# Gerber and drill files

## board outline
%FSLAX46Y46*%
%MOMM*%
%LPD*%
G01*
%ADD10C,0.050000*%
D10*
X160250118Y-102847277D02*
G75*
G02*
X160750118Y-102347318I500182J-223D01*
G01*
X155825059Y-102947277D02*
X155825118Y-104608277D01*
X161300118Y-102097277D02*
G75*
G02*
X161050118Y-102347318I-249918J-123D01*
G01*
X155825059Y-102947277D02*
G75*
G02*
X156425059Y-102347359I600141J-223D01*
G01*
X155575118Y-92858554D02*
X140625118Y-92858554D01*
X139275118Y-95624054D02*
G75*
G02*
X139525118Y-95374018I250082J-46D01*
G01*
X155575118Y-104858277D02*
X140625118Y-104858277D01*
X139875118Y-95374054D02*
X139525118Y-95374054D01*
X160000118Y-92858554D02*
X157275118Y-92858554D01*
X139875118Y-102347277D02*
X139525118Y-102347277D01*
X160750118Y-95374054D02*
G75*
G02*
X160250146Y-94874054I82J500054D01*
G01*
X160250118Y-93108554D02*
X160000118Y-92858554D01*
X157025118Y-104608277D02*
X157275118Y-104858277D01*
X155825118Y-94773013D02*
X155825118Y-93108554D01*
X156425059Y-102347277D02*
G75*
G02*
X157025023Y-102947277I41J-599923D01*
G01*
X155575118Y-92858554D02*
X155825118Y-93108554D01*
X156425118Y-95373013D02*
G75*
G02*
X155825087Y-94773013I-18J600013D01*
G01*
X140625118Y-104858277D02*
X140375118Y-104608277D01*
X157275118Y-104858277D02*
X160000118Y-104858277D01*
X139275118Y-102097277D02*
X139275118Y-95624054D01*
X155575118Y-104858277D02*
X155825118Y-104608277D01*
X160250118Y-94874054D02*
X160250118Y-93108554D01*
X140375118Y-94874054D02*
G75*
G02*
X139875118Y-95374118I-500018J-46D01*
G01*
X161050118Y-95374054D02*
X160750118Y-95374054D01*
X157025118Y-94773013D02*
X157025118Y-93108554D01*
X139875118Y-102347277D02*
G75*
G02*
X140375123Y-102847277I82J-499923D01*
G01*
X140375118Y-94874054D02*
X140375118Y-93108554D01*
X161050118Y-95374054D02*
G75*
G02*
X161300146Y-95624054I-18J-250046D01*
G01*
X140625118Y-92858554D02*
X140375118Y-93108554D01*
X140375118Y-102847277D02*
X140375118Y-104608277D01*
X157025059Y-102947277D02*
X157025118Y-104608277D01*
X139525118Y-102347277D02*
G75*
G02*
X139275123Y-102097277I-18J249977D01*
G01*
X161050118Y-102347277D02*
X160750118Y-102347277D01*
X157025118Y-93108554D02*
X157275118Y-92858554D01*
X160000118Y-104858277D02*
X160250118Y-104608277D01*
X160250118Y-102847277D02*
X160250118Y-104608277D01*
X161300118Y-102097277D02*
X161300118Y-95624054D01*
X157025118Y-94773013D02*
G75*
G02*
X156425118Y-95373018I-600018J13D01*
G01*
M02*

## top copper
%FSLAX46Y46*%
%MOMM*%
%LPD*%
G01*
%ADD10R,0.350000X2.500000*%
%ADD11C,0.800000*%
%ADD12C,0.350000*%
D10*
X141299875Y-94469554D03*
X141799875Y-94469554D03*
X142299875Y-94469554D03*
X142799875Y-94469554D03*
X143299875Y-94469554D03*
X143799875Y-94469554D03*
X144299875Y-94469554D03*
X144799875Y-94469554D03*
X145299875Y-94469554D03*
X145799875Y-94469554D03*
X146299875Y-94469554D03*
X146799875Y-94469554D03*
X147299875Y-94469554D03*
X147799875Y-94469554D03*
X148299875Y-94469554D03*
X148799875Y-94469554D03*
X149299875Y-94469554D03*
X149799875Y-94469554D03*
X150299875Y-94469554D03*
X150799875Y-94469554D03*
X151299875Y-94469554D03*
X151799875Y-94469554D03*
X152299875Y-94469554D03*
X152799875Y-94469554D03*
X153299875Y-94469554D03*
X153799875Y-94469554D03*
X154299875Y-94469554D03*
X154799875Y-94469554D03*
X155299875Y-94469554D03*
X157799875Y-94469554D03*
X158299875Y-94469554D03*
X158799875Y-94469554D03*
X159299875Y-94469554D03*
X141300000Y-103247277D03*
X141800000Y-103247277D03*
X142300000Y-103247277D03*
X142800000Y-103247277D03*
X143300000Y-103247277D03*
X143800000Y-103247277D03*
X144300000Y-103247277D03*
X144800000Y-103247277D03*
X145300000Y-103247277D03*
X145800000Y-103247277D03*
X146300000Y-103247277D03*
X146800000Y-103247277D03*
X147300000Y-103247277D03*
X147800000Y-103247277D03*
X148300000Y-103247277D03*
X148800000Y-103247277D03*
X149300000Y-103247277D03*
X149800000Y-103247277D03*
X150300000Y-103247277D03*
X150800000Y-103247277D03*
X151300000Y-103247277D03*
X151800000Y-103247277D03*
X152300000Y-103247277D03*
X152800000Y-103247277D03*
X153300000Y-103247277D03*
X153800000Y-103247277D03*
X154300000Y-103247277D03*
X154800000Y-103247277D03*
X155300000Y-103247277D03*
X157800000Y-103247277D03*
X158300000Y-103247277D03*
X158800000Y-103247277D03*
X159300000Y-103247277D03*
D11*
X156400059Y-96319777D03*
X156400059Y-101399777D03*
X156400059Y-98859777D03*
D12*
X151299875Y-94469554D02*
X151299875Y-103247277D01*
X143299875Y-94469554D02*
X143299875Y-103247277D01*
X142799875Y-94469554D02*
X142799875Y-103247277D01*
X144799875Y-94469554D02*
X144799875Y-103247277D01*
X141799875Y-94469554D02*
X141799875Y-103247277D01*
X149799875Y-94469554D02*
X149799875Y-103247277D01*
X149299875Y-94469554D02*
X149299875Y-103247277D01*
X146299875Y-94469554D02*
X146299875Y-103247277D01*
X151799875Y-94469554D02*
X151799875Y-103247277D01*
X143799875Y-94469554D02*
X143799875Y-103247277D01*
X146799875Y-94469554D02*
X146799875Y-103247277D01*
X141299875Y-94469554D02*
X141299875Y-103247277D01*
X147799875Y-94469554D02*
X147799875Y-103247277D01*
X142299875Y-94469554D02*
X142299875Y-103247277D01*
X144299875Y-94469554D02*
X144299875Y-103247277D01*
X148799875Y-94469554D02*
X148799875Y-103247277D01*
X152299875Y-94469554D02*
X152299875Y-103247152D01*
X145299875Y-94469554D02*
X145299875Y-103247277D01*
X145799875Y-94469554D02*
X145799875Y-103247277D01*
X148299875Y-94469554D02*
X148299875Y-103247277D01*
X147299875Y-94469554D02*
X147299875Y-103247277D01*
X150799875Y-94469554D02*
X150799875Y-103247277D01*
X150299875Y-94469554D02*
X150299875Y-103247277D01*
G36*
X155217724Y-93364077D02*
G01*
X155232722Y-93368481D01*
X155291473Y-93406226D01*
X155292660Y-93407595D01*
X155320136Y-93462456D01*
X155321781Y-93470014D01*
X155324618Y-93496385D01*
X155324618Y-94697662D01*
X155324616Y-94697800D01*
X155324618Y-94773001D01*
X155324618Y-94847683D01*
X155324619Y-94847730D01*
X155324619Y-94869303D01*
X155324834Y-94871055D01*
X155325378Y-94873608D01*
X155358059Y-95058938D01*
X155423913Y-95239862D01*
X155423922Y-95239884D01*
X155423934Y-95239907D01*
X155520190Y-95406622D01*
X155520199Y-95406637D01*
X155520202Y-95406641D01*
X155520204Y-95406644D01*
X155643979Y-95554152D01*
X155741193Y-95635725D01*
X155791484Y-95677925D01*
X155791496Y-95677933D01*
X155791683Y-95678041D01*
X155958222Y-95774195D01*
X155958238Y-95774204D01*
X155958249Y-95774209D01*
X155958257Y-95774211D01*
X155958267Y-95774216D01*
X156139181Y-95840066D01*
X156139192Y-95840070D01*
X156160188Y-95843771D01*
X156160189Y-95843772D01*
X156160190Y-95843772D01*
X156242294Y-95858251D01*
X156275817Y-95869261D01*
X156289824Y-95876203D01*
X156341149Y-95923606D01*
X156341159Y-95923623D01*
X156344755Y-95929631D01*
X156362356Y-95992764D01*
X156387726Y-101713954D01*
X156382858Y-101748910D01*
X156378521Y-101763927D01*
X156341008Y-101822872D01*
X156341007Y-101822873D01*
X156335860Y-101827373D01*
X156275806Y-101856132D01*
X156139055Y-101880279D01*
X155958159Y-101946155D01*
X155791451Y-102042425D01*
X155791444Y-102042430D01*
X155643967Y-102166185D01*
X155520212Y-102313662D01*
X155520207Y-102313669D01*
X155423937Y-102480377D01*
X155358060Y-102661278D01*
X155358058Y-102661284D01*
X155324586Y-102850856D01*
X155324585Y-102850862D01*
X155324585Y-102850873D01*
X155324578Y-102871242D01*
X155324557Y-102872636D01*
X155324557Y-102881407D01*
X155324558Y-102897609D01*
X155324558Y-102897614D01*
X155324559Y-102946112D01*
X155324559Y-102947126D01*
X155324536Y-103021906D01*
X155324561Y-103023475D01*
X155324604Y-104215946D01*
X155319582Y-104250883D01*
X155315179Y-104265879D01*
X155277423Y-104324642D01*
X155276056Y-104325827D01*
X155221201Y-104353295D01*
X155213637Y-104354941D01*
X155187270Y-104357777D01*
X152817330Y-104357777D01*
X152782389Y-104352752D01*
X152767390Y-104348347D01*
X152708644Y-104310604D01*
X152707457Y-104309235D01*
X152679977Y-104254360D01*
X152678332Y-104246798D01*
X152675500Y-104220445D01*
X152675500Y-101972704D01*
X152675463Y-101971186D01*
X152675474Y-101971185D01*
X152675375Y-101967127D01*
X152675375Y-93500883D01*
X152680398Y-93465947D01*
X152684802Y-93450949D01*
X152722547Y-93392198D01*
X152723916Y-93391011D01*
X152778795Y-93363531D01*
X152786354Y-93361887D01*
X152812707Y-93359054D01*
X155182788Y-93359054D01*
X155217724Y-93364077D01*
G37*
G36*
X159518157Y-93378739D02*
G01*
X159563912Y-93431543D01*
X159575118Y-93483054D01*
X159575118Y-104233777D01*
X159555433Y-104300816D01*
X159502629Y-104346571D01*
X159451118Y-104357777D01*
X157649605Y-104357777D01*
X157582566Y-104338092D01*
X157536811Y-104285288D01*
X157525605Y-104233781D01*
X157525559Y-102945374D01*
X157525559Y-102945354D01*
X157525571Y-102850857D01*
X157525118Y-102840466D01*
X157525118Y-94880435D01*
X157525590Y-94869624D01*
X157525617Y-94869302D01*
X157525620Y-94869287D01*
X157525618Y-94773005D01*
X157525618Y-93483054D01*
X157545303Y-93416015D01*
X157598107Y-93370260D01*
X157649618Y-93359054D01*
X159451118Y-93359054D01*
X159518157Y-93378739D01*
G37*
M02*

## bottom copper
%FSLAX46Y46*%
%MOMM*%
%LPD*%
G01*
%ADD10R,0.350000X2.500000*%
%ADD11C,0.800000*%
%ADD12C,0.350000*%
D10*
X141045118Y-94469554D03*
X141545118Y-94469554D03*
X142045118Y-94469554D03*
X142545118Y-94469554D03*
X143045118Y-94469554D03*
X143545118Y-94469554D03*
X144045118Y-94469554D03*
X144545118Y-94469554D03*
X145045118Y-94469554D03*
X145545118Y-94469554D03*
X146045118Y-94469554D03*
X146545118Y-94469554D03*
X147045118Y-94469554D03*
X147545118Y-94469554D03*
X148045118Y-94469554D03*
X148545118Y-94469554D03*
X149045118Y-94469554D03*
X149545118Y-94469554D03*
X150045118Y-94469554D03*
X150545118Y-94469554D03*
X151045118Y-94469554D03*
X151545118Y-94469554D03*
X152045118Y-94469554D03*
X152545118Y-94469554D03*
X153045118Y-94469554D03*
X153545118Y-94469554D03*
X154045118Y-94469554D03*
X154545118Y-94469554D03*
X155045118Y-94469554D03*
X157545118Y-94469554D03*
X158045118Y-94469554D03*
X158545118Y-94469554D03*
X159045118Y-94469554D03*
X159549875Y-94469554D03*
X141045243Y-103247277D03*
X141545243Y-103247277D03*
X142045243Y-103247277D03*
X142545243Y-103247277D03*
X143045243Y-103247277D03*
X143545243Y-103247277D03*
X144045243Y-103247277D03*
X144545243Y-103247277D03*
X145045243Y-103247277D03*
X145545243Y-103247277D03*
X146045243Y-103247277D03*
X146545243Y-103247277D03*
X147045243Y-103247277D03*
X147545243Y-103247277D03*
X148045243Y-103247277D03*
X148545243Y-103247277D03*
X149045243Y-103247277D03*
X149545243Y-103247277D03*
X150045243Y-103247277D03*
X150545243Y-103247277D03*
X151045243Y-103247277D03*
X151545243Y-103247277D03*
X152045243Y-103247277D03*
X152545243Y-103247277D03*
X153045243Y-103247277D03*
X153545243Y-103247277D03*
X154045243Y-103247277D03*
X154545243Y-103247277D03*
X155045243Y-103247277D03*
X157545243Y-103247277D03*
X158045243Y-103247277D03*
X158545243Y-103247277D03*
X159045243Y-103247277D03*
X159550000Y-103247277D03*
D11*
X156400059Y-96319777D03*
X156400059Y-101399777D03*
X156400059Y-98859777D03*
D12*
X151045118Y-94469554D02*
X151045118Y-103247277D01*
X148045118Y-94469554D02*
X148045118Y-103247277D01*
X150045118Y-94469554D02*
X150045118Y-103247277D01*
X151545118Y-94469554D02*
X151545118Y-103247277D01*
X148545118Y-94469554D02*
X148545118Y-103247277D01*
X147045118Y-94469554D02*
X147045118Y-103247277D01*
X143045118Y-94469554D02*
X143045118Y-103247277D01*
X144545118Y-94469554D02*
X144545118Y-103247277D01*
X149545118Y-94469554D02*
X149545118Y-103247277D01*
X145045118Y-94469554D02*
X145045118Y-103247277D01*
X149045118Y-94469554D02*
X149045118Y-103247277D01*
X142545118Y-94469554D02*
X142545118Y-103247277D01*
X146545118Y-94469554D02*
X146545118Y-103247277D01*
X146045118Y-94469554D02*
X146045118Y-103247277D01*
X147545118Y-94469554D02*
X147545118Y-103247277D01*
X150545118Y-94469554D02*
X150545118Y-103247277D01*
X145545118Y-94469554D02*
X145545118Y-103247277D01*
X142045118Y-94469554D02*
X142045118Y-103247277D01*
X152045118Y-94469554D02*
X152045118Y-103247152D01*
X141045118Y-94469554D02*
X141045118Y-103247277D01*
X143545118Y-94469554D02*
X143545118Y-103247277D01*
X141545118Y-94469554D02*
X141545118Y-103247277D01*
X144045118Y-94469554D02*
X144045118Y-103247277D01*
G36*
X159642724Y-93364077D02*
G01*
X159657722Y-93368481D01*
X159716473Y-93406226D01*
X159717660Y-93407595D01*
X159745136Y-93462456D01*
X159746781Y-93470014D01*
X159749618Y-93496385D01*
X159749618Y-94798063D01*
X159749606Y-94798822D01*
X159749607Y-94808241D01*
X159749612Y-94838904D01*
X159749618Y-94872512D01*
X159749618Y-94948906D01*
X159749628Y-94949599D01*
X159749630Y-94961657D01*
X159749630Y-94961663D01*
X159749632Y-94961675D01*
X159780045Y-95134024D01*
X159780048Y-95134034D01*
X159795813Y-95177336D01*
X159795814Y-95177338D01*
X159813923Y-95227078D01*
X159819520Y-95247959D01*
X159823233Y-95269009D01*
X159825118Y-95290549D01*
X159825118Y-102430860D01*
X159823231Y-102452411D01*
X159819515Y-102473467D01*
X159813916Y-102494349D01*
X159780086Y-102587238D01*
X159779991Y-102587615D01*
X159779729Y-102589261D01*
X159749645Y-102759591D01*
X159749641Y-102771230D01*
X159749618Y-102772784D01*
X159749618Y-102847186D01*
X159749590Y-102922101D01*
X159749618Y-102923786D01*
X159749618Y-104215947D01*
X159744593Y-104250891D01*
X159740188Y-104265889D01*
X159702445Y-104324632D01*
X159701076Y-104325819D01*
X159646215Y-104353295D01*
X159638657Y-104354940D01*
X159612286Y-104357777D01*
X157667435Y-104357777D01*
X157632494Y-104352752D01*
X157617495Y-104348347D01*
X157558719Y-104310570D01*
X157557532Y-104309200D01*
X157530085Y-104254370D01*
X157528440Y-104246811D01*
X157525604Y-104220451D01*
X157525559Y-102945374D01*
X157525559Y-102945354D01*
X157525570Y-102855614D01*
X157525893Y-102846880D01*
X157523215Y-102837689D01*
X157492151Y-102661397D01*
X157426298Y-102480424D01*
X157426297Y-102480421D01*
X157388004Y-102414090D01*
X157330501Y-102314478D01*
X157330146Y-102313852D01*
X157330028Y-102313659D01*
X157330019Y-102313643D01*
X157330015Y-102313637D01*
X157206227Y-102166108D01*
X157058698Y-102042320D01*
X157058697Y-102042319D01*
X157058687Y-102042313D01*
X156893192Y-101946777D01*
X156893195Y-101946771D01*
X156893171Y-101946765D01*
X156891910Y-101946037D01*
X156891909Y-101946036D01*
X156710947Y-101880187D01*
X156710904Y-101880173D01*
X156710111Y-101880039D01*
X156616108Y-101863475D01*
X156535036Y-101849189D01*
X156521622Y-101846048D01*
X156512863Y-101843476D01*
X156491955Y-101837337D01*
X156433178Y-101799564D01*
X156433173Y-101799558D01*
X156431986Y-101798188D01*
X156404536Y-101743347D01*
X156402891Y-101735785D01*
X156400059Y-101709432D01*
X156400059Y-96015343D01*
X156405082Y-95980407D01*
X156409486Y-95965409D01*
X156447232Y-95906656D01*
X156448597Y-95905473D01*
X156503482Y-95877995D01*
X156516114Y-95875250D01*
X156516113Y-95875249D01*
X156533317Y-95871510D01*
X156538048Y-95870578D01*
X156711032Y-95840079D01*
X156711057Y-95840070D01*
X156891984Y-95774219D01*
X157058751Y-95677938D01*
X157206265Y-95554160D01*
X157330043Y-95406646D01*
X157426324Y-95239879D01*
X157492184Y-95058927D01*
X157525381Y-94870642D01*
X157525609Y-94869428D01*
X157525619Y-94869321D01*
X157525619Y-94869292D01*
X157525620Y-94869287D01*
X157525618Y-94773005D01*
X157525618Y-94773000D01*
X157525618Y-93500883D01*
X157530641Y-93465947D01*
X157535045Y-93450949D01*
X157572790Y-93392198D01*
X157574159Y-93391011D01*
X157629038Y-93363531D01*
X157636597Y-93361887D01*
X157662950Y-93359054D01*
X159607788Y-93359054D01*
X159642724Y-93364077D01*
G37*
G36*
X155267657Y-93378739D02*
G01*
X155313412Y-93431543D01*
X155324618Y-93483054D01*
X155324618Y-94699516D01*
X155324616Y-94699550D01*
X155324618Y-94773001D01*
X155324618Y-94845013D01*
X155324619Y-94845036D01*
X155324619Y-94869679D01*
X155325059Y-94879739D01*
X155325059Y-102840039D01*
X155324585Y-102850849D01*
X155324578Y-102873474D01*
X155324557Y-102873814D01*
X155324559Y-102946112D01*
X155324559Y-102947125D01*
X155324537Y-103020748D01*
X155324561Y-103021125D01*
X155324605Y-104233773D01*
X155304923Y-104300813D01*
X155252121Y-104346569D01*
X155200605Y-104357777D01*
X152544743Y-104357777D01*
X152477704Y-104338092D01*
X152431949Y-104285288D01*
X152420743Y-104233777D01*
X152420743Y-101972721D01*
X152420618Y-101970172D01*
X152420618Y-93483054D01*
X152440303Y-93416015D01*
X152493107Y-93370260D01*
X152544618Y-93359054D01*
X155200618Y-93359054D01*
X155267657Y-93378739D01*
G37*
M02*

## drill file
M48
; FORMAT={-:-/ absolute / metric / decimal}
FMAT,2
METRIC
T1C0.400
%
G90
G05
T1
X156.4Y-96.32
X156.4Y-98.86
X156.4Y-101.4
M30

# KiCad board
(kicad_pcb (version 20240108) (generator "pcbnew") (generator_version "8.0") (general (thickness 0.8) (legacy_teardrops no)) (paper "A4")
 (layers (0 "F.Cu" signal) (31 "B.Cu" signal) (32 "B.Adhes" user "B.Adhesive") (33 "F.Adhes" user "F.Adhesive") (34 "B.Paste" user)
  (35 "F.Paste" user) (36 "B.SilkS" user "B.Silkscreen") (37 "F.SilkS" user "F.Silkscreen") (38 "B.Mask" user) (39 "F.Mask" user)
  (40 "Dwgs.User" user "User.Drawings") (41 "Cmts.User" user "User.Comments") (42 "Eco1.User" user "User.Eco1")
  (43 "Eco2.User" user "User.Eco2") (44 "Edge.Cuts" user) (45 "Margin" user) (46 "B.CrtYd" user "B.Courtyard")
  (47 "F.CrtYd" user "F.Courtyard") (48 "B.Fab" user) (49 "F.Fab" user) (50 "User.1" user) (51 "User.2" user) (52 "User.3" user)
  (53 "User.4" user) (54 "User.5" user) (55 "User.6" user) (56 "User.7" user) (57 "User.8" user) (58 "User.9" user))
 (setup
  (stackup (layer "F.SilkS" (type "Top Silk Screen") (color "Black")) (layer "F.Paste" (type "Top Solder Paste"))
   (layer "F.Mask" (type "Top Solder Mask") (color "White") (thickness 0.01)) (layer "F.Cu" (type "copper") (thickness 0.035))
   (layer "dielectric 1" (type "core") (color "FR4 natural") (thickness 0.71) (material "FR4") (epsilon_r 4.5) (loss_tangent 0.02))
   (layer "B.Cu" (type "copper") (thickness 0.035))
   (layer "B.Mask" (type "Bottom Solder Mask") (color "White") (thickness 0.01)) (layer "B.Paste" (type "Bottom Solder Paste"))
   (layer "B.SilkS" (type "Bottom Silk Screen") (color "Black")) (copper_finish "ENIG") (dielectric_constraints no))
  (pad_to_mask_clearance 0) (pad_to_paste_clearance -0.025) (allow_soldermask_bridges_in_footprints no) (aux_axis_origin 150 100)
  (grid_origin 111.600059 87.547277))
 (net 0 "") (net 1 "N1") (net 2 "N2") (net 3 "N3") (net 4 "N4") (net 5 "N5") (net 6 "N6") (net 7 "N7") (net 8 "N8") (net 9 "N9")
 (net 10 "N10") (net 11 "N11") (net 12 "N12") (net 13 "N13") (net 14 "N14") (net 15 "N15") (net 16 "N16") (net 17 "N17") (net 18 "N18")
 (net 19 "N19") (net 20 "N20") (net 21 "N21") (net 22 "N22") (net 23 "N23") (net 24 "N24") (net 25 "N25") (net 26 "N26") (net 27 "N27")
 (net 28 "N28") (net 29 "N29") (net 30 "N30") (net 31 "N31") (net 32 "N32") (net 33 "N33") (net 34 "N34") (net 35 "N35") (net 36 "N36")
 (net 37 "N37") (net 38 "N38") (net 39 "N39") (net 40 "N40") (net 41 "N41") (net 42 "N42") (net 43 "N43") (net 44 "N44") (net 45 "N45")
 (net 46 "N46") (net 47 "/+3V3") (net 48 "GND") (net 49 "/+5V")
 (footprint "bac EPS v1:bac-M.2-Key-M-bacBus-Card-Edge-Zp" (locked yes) (layer "F.Cu") (at 150.349875 96.719554)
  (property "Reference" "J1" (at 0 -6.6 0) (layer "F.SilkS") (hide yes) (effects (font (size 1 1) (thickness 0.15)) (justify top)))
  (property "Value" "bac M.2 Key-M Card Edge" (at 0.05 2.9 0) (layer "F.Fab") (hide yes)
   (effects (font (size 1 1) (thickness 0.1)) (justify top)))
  (pad "1" smd rect (at -9.304757 -2.25) (size 0.35 2.5) (layers "B.Cu" "B.Mask") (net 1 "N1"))
  (pad "2" smd rect (at -9.05 -2.25) (size 0.35 2.5) (layers "F.Cu" "F.Mask") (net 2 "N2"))
  (pad "3" smd rect (at -8.804757 -2.25) (size 0.35 2.5) (layers "B.Cu" "B.Mask") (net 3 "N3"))
  (pad "4" smd rect (at -8.55 -2.25) (size 0.35 2.5) (layers "F.Cu" "F.Mask") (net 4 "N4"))
  (pad "5" smd rect (at -8.304757 -2.25) (size 0.35 2.5) (layers "B.Cu" "B.Mask") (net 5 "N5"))
  (pad "6" smd rect (at -8.05 -2.25) (size 0.35 2.5) (layers "F.Cu" "F.Mask") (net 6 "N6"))
  (pad "7" smd rect (at -7.804757 -2.25) (size 0.35 2.5) (layers "B.Cu" "B.Mask") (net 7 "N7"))
  (pad "8" smd rect (at -7.55 -2.25) (size 0.35 2.5) (layers "F.Cu" "F.Mask") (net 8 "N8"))
  (pad "9" smd rect (at -7.304757 -2.25) (size 0.35 2.5) (layers "B.Cu" "B.Mask") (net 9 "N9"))
  (pad "10" smd rect (at -7.05 -2.25) (size 0.35 2.5) (layers "F.Cu" "F.Mask") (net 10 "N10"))
  (pad "11" smd rect (at -6.804757 -2.25) (size 0.35 2.5) (layers "B.Cu" "B.Mask") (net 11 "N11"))
  (pad "12" smd rect (at -6.55 -2.25) (size 0.35 2.5) (layers "F.Cu" "F.Mask") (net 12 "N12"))
  (pad "13" smd rect (at -6.304757 -2.25) (size 0.35 2.5) (layers "B.Cu" "B.Mask") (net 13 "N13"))
  (pad "14" smd rect (at -6.05 -2.25) (size 0.35 2.5) (layers "F.Cu" "F.Mask") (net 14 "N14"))
  (pad "15" smd rect (at -5.804757 -2.25) (size 0.35 2.5) (layers "B.Cu" "B.Mask") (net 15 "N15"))
  (pad "16" smd rect (at -5.55 -2.25) (size 0.35 2.5) (layers "F.Cu" "F.Mask") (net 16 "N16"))
  (pad "17" smd rect (at -5.304757 -2.25) (size 0.35 2.5) (layers "B.Cu" "B.Mask") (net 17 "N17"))
  (pad "18" smd rect (at -5.05 -2.25) (size 0.35 2.5) (layers "F.Cu" "F.Mask") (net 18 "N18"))
  (pad "19" smd rect (at -4.804757 -2.25) (size 0.35 2.5) (layers "B.Cu" "B.Mask") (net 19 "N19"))
  (pad "20" smd rect (at -4.55 -2.25) (size 0.35 2.5) (layers "F.Cu" "F.Mask") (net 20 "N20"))
  (pad "21" smd rect (at -4.304757 -2.25) (size 0.35 2.5) (layers "B.Cu" "B.Mask") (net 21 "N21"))
  (pad "22" smd rect (at -4.05 -2.25) (size 0.35 2.5) (layers "F.Cu" "F.Mask") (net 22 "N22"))
  (pad "23" smd rect (at -3.804757 -2.25) (size 0.35 2.5) (layers "B.Cu" "B.Mask") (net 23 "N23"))
  (pad "24" smd rect (at -3.55 -2.25) (size 0.35 2.5) (layers "F.Cu" "F.Mask") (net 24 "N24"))
  (pad "25" smd rect (at -3.304757 -2.25) (size 0.35 2.5) (layers "B.Cu" "B.Mask") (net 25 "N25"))
  (pad "26" smd rect (at -3.05 -2.25) (size 0.35 2.5) (layers "F.Cu" "F.Mask") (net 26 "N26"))
  (pad "27" smd rect (at -2.804757 -2.25) (size 0.35 2.5) (layers "B.Cu" "B.Mask") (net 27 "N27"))
  (pad "28" smd rect (at -2.55 -2.25) (size 0.35 2.5) (layers "F.Cu" "F.Mask") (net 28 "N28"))
  (pad "29" smd rect (at -2.304757 -2.25) (size 0.35 2.5) (layers "B.Cu" "B.Mask") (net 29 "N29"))
  (pad "30" smd rect (at -2.05 -2.25) (size 0.35 2.5) (layers "F.Cu" "F.Mask") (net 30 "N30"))
  (pad "31" smd rect (at -1.804757 -2.25) (size 0.35 2.5) (layers "B.Cu" "B.Mask") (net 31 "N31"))
  (pad "32" smd rect (at -1.55 -2.25) (size 0.35 2.5) (layers "F.Cu" "F.Mask") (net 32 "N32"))
  (pad "33" smd rect (at -1.304757 -2.25) (size 0.35 2.5) (layers "B.Cu" "B.Mask") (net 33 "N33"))
  (pad "34" smd rect (at -1.05 -2.25) (size 0.35 2.5) (layers "F.Cu" "F.Mask") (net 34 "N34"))
  (pad "35" smd rect (at -0.804757 -2.25) (size 0.35 2.5) (layers "B.Cu" "B.Mask") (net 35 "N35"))
  (pad "36" smd rect (at -0.55 -2.25) (size 0.35 2.5) (layers "F.Cu" "F.Mask") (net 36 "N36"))
  (pad "37" smd rect (at -0.304757 -2.25) (size 0.35 2.5) (layers "B.Cu" "B.Mask") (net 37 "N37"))
  (pad "38" smd rect (at -0.05 -2.25) (size 0.35 2.5) (layers "F.Cu" "F.Mask") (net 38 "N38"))
  (pad "39" smd rect (at 0.195243 -2.25) (size 0.35 2.5) (layers "B.Cu" "B.Mask") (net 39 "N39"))
  (pad "40" smd rect (at 0.45 -2.25) (size 0.35 2.5) (layers "F.Cu" "F.Mask") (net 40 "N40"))
  (pad "41" smd rect (at 0.695243 -2.25) (size 0.35 2.5) (layers "B.Cu" "B.Mask") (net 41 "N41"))
  (pad "42" smd rect (at 0.95 -2.25) (size 0.35 2.5) (layers "F.Cu" "F.Mask") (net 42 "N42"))
  (pad "43" smd rect (at 1.195243 -2.25) (size 0.35 2.5) (layers "B.Cu" "B.Mask") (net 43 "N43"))
  (pad "44" smd rect (at 1.45 -2.25) (size 0.35 2.5) (layers "F.Cu" "F.Mask") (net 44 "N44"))
  (pad "45" smd rect (at 1.695243 -2.25) (size 0.35 2.5) (layers "B.Cu" "B.Mask") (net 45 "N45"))
  (pad "46" smd rect (at 1.95 -2.25) (size 0.35 2.5) (layers "F.Cu" "F.Mask") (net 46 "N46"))
  (pad "47" smd rect (at 2.195243 -2.25) (size 0.35 2.5) (layers "B.Cu" "B.Mask") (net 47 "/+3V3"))
  (pad "48" smd rect (at 2.45 -2.25) (size 0.35 2.5) (layers "F.Cu" "F.Mask") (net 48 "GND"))
  (pad "49" smd rect (at 2.695243 -2.25) (size 0.35 2.5) (layers "B.Cu" "B.Mask") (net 47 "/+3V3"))
  (pad "50" smd rect (at 2.95 -2.25) (size 0.35 2.5) (layers "F.Cu" "F.Mask") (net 48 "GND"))
  (pad "51" smd rect (at 3.195243 -2.25) (size 0.35 2.5) (layers "B.Cu" "B.Mask") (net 47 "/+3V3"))
  (pad "52" smd rect (at 3.45 -2.25) (size 0.35 2.5) (layers "F.Cu" "F.Mask") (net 48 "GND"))
  (pad "53" smd rect (at 3.695243 -2.25) (size 0.35 2.5) (layers "B.Cu" "B.Mask") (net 47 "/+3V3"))
  (pad "54" smd rect (at 3.95 -2.25) (size 0.35 2.5) (layers "F.Cu" "F.Mask") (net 48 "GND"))
  (pad "55" smd rect (at 4.195243 -2.25) (size 0.35 2.5) (layers "B.Cu" "B.Mask") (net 47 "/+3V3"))
  (pad "56" smd rect (at 4.45 -2.25) (size 0.35 2.5) (layers "F.Cu" "F.Mask") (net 48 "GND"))
  (pad "57" smd rect (at 4.695243 -2.25) (size 0.35 2.5) (layers "B.Cu" "B.Mask") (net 47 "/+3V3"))
  (pad "58" smd rect (at 4.95 -2.25) (size 0.35 2.5) (layers "F.Cu" "F.Mask") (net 48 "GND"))
  (pad "67" smd rect (at 7.195243 -2.25) (size 0.35 2.5) (layers "B.Cu" "B.Mask") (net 48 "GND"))
  (pad "68" smd rect (at 7.45 -2.25) (size 0.35 2.5) (layers "F.Cu" "F.Mask") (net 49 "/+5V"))
  (pad "69" smd rect (at 7.695243 -2.25) (size 0.35 2.5) (layers "B.Cu" "B.Mask") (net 48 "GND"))
  (pad "70" smd rect (at 7.95 -2.25) (size 0.35 2.5) (layers "F.Cu" "F.Mask") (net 49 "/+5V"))
  (pad "71" smd rect (at 8.195243 -2.25) (size 0.35 2.5) (layers "B.Cu" "B.Mask") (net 48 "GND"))
  (pad "72" smd rect (at 8.45 -2.25) (size 0.35 2.5) (layers "F.Cu" "F.Mask") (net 49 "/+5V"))
  (pad "73" smd rect (at 8.695243 -2.25) (size 0.35 2.5) (layers "B.Cu" "B.Mask") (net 48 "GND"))
  (pad "74" smd rect (at 8.95 -2.25) (size 0.35 2.5) (layers "F.Cu" "F.Mask") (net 49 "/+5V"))
  (pad "75" smd rect (at 9.2 -2.25) (size 0.35 2.5) (layers "B.Cu" "B.Mask") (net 48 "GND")))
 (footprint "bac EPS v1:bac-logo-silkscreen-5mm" (layer "F.Cu") (at 150.050059 98.947277)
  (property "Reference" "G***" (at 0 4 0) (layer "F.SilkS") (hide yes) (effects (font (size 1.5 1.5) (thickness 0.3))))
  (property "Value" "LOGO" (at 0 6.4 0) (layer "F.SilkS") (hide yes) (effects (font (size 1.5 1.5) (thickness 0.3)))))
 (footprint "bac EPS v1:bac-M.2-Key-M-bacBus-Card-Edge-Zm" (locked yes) (layer "F.Cu") (at 150.15 105.197277)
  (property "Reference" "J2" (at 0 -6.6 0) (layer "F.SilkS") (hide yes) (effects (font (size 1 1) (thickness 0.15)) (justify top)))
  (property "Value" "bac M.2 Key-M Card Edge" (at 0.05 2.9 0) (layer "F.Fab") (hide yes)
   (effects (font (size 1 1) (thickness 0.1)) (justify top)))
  (pad "1" smd rect (at -9.104757 -1.95 180) (size 0.35 2.5) (layers "B.Cu" "B.Mask") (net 1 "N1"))
  (pad "2" smd rect (at -8.85 -1.95 180) (size 0.35 2.5) (layers "F.Cu" "F.Mask") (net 2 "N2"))
  (pad "3" smd rect (at -8.604757 -1.95 180) (size 0.35 2.5) (layers "B.Cu" "B.Mask") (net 3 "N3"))
  (pad "4" smd rect (at -8.35 -1.95 180) (size 0.35 2.5) (layers "F.Cu" "F.Mask") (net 4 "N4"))
  (pad "5" smd rect (at -8.104757 -1.95 180) (size 0.35 2.5) (layers "B.Cu" "B.Mask") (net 5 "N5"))
  (pad "6" smd rect (at -7.85 -1.95 180) (size 0.35 2.5) (layers "F.Cu" "F.Mask") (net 6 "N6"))
  (pad "7" smd rect (at -7.604757 -1.95 180) (size 0.35 2.5) (layers "B.Cu" "B.Mask") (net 7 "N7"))
  (pad "8" smd rect (at -7.35 -1.95 180) (size 0.35 2.5) (layers "F.Cu" "F.Mask") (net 8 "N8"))
  (pad "9" smd rect (at -7.104757 -1.95 180) (size 0.35 2.5) (layers "B.Cu" "B.Mask") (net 9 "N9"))
  (pad "10" smd rect (at -6.85 -1.95 180) (size 0.35 2.5) (layers "F.Cu" "F.Mask") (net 10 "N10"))
  (pad "11" smd rect (at -6.604757 -1.95 180) (size 0.35 2.5) (layers "B.Cu" "B.Mask") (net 11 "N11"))
  (pad "12" smd rect (at -6.35 -1.95 180) (size 0.35 2.5) (layers "F.Cu" "F.Mask") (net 12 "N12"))
  (pad "13" smd rect (at -6.104757 -1.95 180) (size 0.35 2.5) (layers "B.Cu" "B.Mask") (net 13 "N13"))
  (pad "14" smd rect (at -5.85 -1.95 180) (size 0.35 2.5) (layers "F.Cu" "F.Mask") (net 14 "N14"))
  (pad "15" smd rect (at -5.604757 -1.95 180) (size 0.35 2.5) (layers "B.Cu" "B.Mask") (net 15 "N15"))
  (pad "16" smd rect (at -5.35 -1.95 180) (size 0.35 2.5) (layers "F.Cu" "F.Mask") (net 16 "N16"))
  (pad "17" smd rect (at -5.104757 -1.95 180) (size 0.35 2.5) (layers "B.Cu" "B.Mask") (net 17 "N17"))
  (pad "18" smd rect (at -4.85 -1.95 180) (size 0.35 2.5) (layers "F.Cu" "F.Mask") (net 18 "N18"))
  (pad "19" smd rect (at -4.604757 -1.95 180) (size 0.35 2.5) (layers "B.Cu" "B.Mask") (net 19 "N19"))
  (pad "20" smd rect (at -4.35 -1.95 180) (size 0.35 2.5) (layers "F.Cu" "F.Mask") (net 20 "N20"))
  (pad "21" smd rect (at -4.104757 -1.95 180) (size 0.35 2.5) (layers "B.Cu" "B.Mask") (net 21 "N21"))
  (pad "22" smd rect (at -3.85 -1.95 180) (size 0.35 2.5) (layers "F.Cu" "F.Mask") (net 22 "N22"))
  (pad "23" smd rect (at -3.604757 -1.95 180) (size 0.35 2.5) (layers "B.Cu" "B.Mask") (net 23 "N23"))
  (pad "24" smd rect (at -3.35 -1.95 180) (size 0.35 2.5) (layers "F.Cu" "F.Mask") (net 24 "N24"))
  (pad "25" smd rect (at -3.104757 -1.95 180) (size 0.35 2.5) (layers "B.Cu" "B.Mask") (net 25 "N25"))
  (pad "26" smd rect (at -2.85 -1.95 180) (size 0.35 2.5) (layers "F.Cu" "F.Mask") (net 26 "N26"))
  (pad "27" smd rect (at -2.604757 -1.95 180) (size 0.35 2.5) (layers "B.Cu" "B.Mask") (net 27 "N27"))
  (pad "28" smd rect (at -2.35 -1.95 180) (size 0.35 2.5) (layers "F.Cu" "F.Mask") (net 28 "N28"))
  (pad "29" smd rect (at -2.104757 -1.95 180) (size 0.35 2.5) (layers "B.Cu" "B.Mask") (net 29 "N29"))
  (pad "30" smd rect (at -1.85 -1.95 180) (size 0.35 2.5) (layers "F.Cu" "F.Mask") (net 30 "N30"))
  (pad "31" smd rect (at -1.604757 -1.95 180) (size 0.35 2.5) (layers "B.Cu" "B.Mask") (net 31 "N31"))
  (pad "32" smd rect (at -1.35 -1.95 180) (size 0.35 2.5) (layers "F.Cu" "F.Mask") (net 32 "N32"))
  (pad "33" smd rect (at -1.104757 -1.95 180) (size 0.35 2.5) (layers "B.Cu" "B.Mask") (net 33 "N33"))
  (pad "34" smd rect (at -0.85 -1.95 180) (size 0.35 2.5) (layers "F.Cu" "F.Mask") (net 34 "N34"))
  (pad "35" smd rect (at -0.604757 -1.95 180) (size 0.35 2.5) (layers "B.Cu" "B.Mask") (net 35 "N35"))
  (pad "36" smd rect (at -0.35 -1.95 180) (size 0.35 2.5) (layers "F.Cu" "F.Mask") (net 36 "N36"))
  (pad "37" smd rect (at -0.104757 -1.95 180) (size 0.35 2.5) (layers "B.Cu" "B.Mask") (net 37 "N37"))
  (pad "38" smd rect (at 0.15 -1.95 180) (size 0.35 2.5) (layers "F.Cu" "F.Mask") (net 38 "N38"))
  (pad "39" smd rect (at 0.395243 -1.95 180) (size 0.35 2.5) (layers "B.Cu" "B.Mask") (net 39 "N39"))
  (pad "40" smd rect (at 0.65 -1.95 180) (size 0.35 2.5) (layers "F.Cu" "F.Mask") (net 40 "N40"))
  (pad "41" smd rect (at 0.895243 -1.95 180) (size 0.35 2.5) (layers "B.Cu" "B.Mask") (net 41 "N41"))
  (pad "42" smd rect (at 1.15 -1.95 180) (size 0.35 2.5) (layers "F.Cu" "F.Mask") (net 42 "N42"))
  (pad "43" smd rect (at 1.395243 -1.95 180) (size 0.35 2.5) (layers "B.Cu" "B.Mask") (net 43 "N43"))
  (pad "44" smd rect (at 1.65 -1.95 180) (size 0.35 2.5) (layers "F.Cu" "F.Mask") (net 44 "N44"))
  (pad "45" smd rect (at 1.895243 -1.95 180) (size 0.35 2.5) (layers "B.Cu" "B.Mask") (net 45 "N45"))
  (pad "46" smd rect (at 2.15 -1.95 180) (size 0.35 2.5) (layers "F.Cu" "F.Mask") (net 46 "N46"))
  (pad "47" smd rect (at 2.395243 -1.95 180) (size 0.35 2.5) (layers "B.Cu" "B.Mask") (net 47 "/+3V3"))
  (pad "48" smd rect (at 2.65 -1.95 180) (size 0.35 2.5) (layers "F.Cu" "F.Mask") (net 48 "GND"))
  (pad "49" smd rect (at 2.895243 -1.95 180) (size 0.35 2.5) (layers "B.Cu" "B.Mask") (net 47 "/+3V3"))
  (pad "50" smd rect (at 3.15 -1.95 180) (size 0.35 2.5) (layers "F.Cu" "F.Mask") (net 48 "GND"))
  (pad "51" smd rect (at 3.395243 -1.95 180) (size 0.35 2.5) (layers "B.Cu" "B.Mask") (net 47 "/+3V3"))
  (pad "52" smd rect (at 3.65 -1.95 180) (size 0.35 2.5) (layers "F.Cu" "F.Mask") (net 48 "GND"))
  (pad "53" smd rect (at 3.895243 -1.95 180) (size 0.35 2.5) (layers "B.Cu" "B.Mask") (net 47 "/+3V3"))
  (pad "54" smd rect (at 4.15 -1.95 180) (size 0.35 2.5) (layers "F.Cu" "F.Mask") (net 48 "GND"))
  (pad "55" smd rect (at 4.395243 -1.95 180) (size 0.35 2.5) (layers "B.Cu" "B.Mask") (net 47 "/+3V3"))
  (pad "56" smd rect (at 4.65 -1.95 180) (size 0.35 2.5) (layers "F.Cu" "F.Mask") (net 48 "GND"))
  (pad "57" smd rect (at 4.895243 -1.95 180) (size 0.35 2.5) (layers "B.Cu" "B.Mask") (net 47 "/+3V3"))
  (pad "58" smd rect (at 5.15 -1.95 180) (size 0.35 2.5) (layers "F.Cu" "F.Mask") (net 48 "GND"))
  (pad "67" smd rect (at 7.395243 -1.95 180) (size 0.35 2.5) (layers "B.Cu" "B.Mask") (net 48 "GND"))
  (pad "68" smd rect (at 7.65 -1.95 180) (size 0.35 2.5) (layers "F.Cu" "F.Mask") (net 49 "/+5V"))
  (pad "69" smd rect (at 7.895243 -1.95 180) (size 0.35 2.5) (layers "B.Cu" "B.Mask") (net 48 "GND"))
  (pad "70" smd rect (at 8.15 -1.95 180) (size 0.35 2.5) (layers "F.Cu" "F.Mask") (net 49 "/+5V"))
  (pad "71" smd rect (at 8.395243 -1.95 180) (size 0.35 2.5) (layers "B.Cu" "B.Mask") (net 48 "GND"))
  (pad "72" smd rect (at 8.65 -1.95 180) (size 0.35 2.5) (layers "F.Cu" "F.Mask") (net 49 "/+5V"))
  (pad "73" smd rect (at 8.895243 -1.95 180) (size 0.35 2.5) (layers "B.Cu" "B.Mask") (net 48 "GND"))
  (pad "74" smd rect (at 9.15 -1.95 180) (size 0.35 2.5) (layers "F.Cu" "F.Mask") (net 49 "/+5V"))
  (pad "75" smd rect (at 9.4 -1.95 180) (size 0.35 2.5) (layers "B.Cu" "B.Mask") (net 48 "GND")))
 (gr_arc (start 160.250118 102.847277) (mid 160.396606 102.493789) (end 160.750118 102.347277) (stroke (width 0.05) (type default))
  (layer "Edge.Cuts"))
 (gr_line (start 155.825059 102.947277) (end 155.825118 104.608277) (stroke (width 0.05) (type default)) (layer "Edge.Cuts"))
 (gr_arc (start 161.300118 102.097277) (mid 161.226912 102.27409) (end 161.050118 102.347277) (stroke (width 0.05) (type default))
  (layer "Edge.Cuts"))
 (gr_arc (start 155.825059 102.947277) (mid 156.000836 102.523078) (end 156.425059 102.347277) (stroke (width 0.05) (type default))
  (layer "Edge.Cuts"))
 (gr_line (start 155.575118 92.858554) (end 140.625118 92.858554) (stroke (width 0.05) (type default)) (layer "Edge.Cuts"))
 (gr_arc (start 139.275118 95.624054) (mid 139.348359 95.447313) (end 139.525118 95.374054) (stroke (width 0.05) (type default))
  (layer "Edge.Cuts"))
 (gr_line (start 155.575118 104.858277) (end 140.625118 104.858277) (stroke (width 0.05) (type default)) (layer "Edge.Cuts"))
 (gr_line (start 139.875118 95.374054) (end 139.525118 95.374054) (stroke (width 0.05) (type default)) (layer "Edge.Cuts"))
 (gr_line (start 160.000118 92.858554) (end 157.275118 92.858554) (stroke (width 0.05) (type default)) (layer "Edge.Cuts"))
 (gr_line (start 139.875118 102.347277) (end 139.525118 102.347277) (stroke (width 0.05) (type default)) (layer "Edge.Cuts"))
 (gr_arc (start 160.750118 95.374054) (mid 160.396599 95.227592) (end 160.250118 94.874054) (stroke (width 0.05) (type default))
  (layer "Edge.Cuts"))
 (gr_line (start 160.250118 93.108554) (end 160.000118 92.858554) (stroke (width 0.05) (type default)) (layer "Edge.Cuts"))
 (gr_line (start 157.025118 104.608277) (end 157.275118 104.858277) (stroke (width 0.05) (type default)) (layer "Edge.Cuts"))
 (gr_line (start 155.825118 94.773013) (end 155.825118 93.108554) (stroke (width 0.05) (type default)) (layer "Edge.Cuts"))
 (gr_arc (start 156.425059 102.347277) (mid 156.849358 102.522997) (end 157.025059 102.947277) (stroke (width 0.05) (type default))
  (layer "Edge.Cuts"))
 (gr_line (start 155.575118 92.858554) (end 155.825118 93.108554) (stroke (width 0.05) (type default)) (layer "Edge.Cuts"))
 (gr_arc (start 156.425118 95.373013) (mid 156.000853 95.197267) (end 155.825118 94.773013) (stroke (width 0.05) (type default))
  (layer "Edge.Cuts"))
 (gr_line (start 140.625118 104.858277) (end 140.375118 104.608277) (stroke (width 0.05) (type default)) (layer "Edge.Cuts"))
 (gr_line (start 157.275118 104.858277) (end 160.000118 104.858277) (stroke (width 0.05) (type default)) (layer "Edge.Cuts"))
 (gr_line (start 139.275118 102.097277) (end 139.275118 95.624054) (stroke (width 0.05) (type default)) (layer "Edge.Cuts"))
 (gr_line (start 155.575118 104.858277) (end 155.825118 104.608277) (stroke (width 0.05) (type default)) (layer "Edge.Cuts"))
 (gr_line (start 160.250118 94.874054) (end 160.250118 93.108554) (stroke (width 0.05) (type default)) (layer "Edge.Cuts"))
 (gr_arc (start 140.375118 94.874054) (mid 140.228677 95.227608) (end 139.875118 95.374054) (stroke (width 0.05) (type default))
  (layer "Edge.Cuts"))
 (gr_line (start 161.050118 95.374054) (end 160.750118 95.374054) (stroke (width 0.05) (type default)) (layer "Edge.Cuts"))
 (gr_line (start 157.025118 94.773013) (end 157.025118 93.108554) (stroke (width 0.05) (type default)) (layer "Edge.Cuts"))
 (gr_arc (start 139.875118 102.347277) (mid 140.228706 102.493708) (end 140.375118 102.847277) (stroke (width 0.05) (type default))
  (layer "Edge.Cuts"))
 (gr_line (start 140.375118 94.874054) (end 140.375118 93.108554) (stroke (width 0.05) (type default)) (layer "Edge.Cuts"))
 (gr_arc (start 161.050118 95.374054) (mid 161.226895 95.447277) (end 161.300118 95.624054) (stroke (width 0.05) (type default))
  (layer "Edge.Cuts"))
 (gr_line (start 140.625118 92.858554) (end 140.375118 93.108554) (stroke (width 0.05) (type default)) (layer "Edge.Cuts"))
 (gr_line (start 140.375118 102.847277) (end 140.375118 104.608277) (stroke (width 0.05) (type default)) (layer "Edge.Cuts"))
 (gr_line (start 157.025059 102.947277) (end 157.025118 104.608277) (stroke (width 0.05) (type default)) (layer "Edge.Cuts"))
 (gr_arc (start 139.525118 102.347277) (mid 139.348346 102.274057) (end 139.275118 102.097277) (stroke (width 0.05) (type default))
  (layer "Edge.Cuts"))
 (gr_line (start 161.050118 102.347277) (end 160.750118 102.347277) (stroke (width 0.05) (type default)) (layer "Edge.Cuts"))
 (gr_line (start 157.025118 93.108554) (end 157.275118 92.858554) (stroke (width 0.05) (type default)) (layer "Edge.Cuts"))
 (gr_line (start 160.000118 104.858277) (end 160.250118 104.608277) (stroke (width 0.05) (type default)) (layer "Edge.Cuts"))
 (gr_line (start 160.250118 102.847277) (end 160.250118 104.608277) (stroke (width 0.05) (type default)) (layer "Edge.Cuts"))
 (gr_line (start 161.300118 102.097277) (end 161.300118 95.624054) (stroke (width 0.05) (type default)) (layer "Edge.Cuts"))
 (gr_arc (start 157.025118 94.773013) (mid 156.849388 95.197277) (end 156.425118 95.373013) (stroke (width 0.05) (type default))
  (layer "Edge.Cuts"))
 (via (at 156.400059 96.319777) (size 0.8) (drill 0.4) (layers "F.Cu" "B.Cu") (free yes) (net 48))
 (via (at 156.400059 101.399777) (size 0.8) (drill 0.4) (layers "F.Cu" "B.Cu") (free yes) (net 48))
 (via (at 156.400059 98.859777) (size 0.8) (drill 0.4) (layers "F.Cu" "B.Cu") (free yes) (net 48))
 (segment (start 151.045118 94.469554) (end 151.045118 103.247277) (width 0.35) (layer "B.Cu") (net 41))
 (segment (start 148.045118 94.469554) (end 148.045118 103.247277) (width 0.35) (layer "B.Cu") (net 29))
 (segment (start 150.045118 94.469554) (end 150.045118 103.247277) (width 0.35) (layer "B.Cu") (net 37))
 (segment (start 151.545118 94.469554) (end 151.545118 103.247277) (width 0.35) (layer "B.Cu") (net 43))
 (segment (start 151.299875 94.469554) (end 151.299875 103.247277) (width 0.35) (layer "F.Cu") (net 42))
 (segment (start 148.545118 94.469554) (end 148.545118 103.247277) (width 0.35) (layer "B.Cu") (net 31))
 (segment (start 143.299875 94.469554) (end 143.299875 103.247277) (width 0.35) (layer "F.Cu") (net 10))
 (segment (start 147.045118 94.469554) (end 147.045118 103.247277) (width 0.35) (layer "B.Cu") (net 25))
 (segment (start 143.045118 94.469554) (end 143.045118 103.247277) (width 0.35) (layer "B.Cu") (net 9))
 (segment (start 142.799875 94.469554) (end 142.799875 103.247277) (width 0.35) (layer "F.Cu") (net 8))
 (segment (start 144.799875 94.469554) (end 144.799875 103.247277) (width 0.35) (layer "F.Cu") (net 16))
 (segment (start 144.545118 94.469554) (end 144.545118 103.247277) (width 0.35) (layer "B.Cu") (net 15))
 (segment (start 141.799875 94.469554) (end 141.799875 103.247277) (width 0.35) (layer "F.Cu") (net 4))
 (segment (start 149.799875 94.469554) (end 149.799875 103.247277) (width 0.35) (layer "F.Cu") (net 36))
 (segment (start 149.545118 94.469554) (end 149.545118 103.247277) (width 0.35) (layer "B.Cu") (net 35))
 (segment (start 145.045118 94.469554) (end 145.045118 103.247277) (width 0.35) (layer "B.Cu") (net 17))
 (segment (start 149.045118 94.469554) (end 149.045118 103.247277) (width 0.35) (layer "B.Cu") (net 33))
 (segment (start 142.545118 94.469554) (end 142.545118 103.247277) (width 0.35) (layer "B.Cu") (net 7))
 (segment (start 149.299875 94.469554) (end 149.299875 103.247277) (width 0.35) (layer "F.Cu") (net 34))
 (segment (start 146.299875 94.469554) (end 146.299875 103.247277) (width 0.35) (layer "F.Cu") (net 22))
 (segment (start 151.799875 94.469554) (end 151.799875 103.247277) (width 0.35) (layer "F.Cu") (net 44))
 (segment (start 143.799875 94.469554) (end 143.799875 103.247277) (width 0.35) (layer "F.Cu") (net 12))
 (segment (start 146.799875 94.469554) (end 146.799875 103.247277) (width 0.35) (layer "F.Cu") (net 24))
 (segment (start 141.299875 94.469554) (end 141.299875 103.247277) (width 0.35) (layer "F.Cu") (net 2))
 (segment (start 146.545118 94.469554) (end 146.545118 103.247277) (width 0.35) (layer "B.Cu") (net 23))
 (segment (start 146.045118 94.469554) (end 146.045118 103.247277) (width 0.35) (layer "B.Cu") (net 21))
 (segment (start 147.799875 94.469554) (end 147.799875 103.247277) (width 0.35) (layer "F.Cu") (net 28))
 (segment (start 147.545118 94.469554) (end 147.545118 103.247277) (width 0.35) (layer "B.Cu") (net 27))
 (segment (start 150.545118 94.469554) (end 150.545118 103.247277) (width 0.35) (layer "B.Cu") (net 39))
 (segment (start 142.299875 94.469554) (end 142.299875 103.247277) (width 0.35) (layer "F.Cu") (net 6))
 (segment (start 145.545118 94.469554) (end 145.545118 103.247277) (width 0.35) (layer "B.Cu") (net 19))
 (segment (start 142.045118 94.469554) (end 142.045118 103.247277) (width 0.35) (layer "B.Cu") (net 5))
 (segment (start 144.299875 94.469554) (end 144.299875 103.247277) (width 0.35) (layer "F.Cu") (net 14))
 (segment (start 152.045118 94.469554) (end 152.045118 103.247152) (width 0.35) (layer "B.Cu") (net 45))
 (segment (start 148.799875 94.469554) (end 148.799875 103.247277) (width 0.35) (layer "F.Cu") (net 32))
 (segment (start 141.045118 94.469554) (end 141.045118 103.247277) (width 0.35) (layer "B.Cu") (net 1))
 (segment (start 152.299875 94.469554) (end 152.299875 103.247152) (width 0.35) (layer "F.Cu") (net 46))
 (segment (start 143.545118 94.469554) (end 143.545118 103.247277) (width 0.35) (layer "B.Cu") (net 11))
 (segment (start 145.299875 94.469554) (end 145.299875 103.247277) (width 0.35) (layer "F.Cu") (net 18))
 (segment (start 145.799875 94.469554) (end 145.799875 103.247277) (width 0.35) (layer "F.Cu") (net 20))
 (segment (start 148.299875 94.469554) (end 148.299875 103.247277) (width 0.35) (layer "F.Cu") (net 30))
 (segment (start 141.545118 94.469554) (end 141.545118 103.247277) (width 0.35) (layer "B.Cu") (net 3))
 (segment (start 147.299875 94.469554) (end 147.299875 103.247277) (width 0.35) (layer "F.Cu") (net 26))
 (segment (start 150.799875 94.469554) (end 150.799875 103.247277) (width 0.35) (layer "F.Cu") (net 40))
 (segment (start 150.299875 94.469554) (end 150.299875 103.247277) (width 0.35) (layer "F.Cu") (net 38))
 (segment (start 144.045118 94.469554) (end 144.045118 103.247277) (width 0.35) (layer "B.Cu") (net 13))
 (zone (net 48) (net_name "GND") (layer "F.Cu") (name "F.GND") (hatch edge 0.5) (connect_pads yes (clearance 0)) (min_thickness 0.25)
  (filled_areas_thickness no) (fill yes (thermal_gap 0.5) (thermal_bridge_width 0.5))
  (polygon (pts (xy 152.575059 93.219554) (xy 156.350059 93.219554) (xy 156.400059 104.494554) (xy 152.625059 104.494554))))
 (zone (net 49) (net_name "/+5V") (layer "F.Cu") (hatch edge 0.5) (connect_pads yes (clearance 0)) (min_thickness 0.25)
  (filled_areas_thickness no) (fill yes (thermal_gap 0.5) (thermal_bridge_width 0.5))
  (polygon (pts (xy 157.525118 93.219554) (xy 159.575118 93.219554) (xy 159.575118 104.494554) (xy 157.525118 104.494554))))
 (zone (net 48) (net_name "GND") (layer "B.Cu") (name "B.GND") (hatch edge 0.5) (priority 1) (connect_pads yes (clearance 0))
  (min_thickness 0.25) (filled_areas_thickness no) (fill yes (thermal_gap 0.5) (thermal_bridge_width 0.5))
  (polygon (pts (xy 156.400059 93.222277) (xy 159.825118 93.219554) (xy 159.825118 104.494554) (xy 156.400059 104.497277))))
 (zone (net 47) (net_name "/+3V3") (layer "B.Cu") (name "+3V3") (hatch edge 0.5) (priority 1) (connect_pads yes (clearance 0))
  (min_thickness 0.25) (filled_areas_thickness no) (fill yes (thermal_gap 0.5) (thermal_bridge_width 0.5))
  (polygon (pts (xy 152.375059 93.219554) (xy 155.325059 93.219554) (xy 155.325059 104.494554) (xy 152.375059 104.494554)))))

